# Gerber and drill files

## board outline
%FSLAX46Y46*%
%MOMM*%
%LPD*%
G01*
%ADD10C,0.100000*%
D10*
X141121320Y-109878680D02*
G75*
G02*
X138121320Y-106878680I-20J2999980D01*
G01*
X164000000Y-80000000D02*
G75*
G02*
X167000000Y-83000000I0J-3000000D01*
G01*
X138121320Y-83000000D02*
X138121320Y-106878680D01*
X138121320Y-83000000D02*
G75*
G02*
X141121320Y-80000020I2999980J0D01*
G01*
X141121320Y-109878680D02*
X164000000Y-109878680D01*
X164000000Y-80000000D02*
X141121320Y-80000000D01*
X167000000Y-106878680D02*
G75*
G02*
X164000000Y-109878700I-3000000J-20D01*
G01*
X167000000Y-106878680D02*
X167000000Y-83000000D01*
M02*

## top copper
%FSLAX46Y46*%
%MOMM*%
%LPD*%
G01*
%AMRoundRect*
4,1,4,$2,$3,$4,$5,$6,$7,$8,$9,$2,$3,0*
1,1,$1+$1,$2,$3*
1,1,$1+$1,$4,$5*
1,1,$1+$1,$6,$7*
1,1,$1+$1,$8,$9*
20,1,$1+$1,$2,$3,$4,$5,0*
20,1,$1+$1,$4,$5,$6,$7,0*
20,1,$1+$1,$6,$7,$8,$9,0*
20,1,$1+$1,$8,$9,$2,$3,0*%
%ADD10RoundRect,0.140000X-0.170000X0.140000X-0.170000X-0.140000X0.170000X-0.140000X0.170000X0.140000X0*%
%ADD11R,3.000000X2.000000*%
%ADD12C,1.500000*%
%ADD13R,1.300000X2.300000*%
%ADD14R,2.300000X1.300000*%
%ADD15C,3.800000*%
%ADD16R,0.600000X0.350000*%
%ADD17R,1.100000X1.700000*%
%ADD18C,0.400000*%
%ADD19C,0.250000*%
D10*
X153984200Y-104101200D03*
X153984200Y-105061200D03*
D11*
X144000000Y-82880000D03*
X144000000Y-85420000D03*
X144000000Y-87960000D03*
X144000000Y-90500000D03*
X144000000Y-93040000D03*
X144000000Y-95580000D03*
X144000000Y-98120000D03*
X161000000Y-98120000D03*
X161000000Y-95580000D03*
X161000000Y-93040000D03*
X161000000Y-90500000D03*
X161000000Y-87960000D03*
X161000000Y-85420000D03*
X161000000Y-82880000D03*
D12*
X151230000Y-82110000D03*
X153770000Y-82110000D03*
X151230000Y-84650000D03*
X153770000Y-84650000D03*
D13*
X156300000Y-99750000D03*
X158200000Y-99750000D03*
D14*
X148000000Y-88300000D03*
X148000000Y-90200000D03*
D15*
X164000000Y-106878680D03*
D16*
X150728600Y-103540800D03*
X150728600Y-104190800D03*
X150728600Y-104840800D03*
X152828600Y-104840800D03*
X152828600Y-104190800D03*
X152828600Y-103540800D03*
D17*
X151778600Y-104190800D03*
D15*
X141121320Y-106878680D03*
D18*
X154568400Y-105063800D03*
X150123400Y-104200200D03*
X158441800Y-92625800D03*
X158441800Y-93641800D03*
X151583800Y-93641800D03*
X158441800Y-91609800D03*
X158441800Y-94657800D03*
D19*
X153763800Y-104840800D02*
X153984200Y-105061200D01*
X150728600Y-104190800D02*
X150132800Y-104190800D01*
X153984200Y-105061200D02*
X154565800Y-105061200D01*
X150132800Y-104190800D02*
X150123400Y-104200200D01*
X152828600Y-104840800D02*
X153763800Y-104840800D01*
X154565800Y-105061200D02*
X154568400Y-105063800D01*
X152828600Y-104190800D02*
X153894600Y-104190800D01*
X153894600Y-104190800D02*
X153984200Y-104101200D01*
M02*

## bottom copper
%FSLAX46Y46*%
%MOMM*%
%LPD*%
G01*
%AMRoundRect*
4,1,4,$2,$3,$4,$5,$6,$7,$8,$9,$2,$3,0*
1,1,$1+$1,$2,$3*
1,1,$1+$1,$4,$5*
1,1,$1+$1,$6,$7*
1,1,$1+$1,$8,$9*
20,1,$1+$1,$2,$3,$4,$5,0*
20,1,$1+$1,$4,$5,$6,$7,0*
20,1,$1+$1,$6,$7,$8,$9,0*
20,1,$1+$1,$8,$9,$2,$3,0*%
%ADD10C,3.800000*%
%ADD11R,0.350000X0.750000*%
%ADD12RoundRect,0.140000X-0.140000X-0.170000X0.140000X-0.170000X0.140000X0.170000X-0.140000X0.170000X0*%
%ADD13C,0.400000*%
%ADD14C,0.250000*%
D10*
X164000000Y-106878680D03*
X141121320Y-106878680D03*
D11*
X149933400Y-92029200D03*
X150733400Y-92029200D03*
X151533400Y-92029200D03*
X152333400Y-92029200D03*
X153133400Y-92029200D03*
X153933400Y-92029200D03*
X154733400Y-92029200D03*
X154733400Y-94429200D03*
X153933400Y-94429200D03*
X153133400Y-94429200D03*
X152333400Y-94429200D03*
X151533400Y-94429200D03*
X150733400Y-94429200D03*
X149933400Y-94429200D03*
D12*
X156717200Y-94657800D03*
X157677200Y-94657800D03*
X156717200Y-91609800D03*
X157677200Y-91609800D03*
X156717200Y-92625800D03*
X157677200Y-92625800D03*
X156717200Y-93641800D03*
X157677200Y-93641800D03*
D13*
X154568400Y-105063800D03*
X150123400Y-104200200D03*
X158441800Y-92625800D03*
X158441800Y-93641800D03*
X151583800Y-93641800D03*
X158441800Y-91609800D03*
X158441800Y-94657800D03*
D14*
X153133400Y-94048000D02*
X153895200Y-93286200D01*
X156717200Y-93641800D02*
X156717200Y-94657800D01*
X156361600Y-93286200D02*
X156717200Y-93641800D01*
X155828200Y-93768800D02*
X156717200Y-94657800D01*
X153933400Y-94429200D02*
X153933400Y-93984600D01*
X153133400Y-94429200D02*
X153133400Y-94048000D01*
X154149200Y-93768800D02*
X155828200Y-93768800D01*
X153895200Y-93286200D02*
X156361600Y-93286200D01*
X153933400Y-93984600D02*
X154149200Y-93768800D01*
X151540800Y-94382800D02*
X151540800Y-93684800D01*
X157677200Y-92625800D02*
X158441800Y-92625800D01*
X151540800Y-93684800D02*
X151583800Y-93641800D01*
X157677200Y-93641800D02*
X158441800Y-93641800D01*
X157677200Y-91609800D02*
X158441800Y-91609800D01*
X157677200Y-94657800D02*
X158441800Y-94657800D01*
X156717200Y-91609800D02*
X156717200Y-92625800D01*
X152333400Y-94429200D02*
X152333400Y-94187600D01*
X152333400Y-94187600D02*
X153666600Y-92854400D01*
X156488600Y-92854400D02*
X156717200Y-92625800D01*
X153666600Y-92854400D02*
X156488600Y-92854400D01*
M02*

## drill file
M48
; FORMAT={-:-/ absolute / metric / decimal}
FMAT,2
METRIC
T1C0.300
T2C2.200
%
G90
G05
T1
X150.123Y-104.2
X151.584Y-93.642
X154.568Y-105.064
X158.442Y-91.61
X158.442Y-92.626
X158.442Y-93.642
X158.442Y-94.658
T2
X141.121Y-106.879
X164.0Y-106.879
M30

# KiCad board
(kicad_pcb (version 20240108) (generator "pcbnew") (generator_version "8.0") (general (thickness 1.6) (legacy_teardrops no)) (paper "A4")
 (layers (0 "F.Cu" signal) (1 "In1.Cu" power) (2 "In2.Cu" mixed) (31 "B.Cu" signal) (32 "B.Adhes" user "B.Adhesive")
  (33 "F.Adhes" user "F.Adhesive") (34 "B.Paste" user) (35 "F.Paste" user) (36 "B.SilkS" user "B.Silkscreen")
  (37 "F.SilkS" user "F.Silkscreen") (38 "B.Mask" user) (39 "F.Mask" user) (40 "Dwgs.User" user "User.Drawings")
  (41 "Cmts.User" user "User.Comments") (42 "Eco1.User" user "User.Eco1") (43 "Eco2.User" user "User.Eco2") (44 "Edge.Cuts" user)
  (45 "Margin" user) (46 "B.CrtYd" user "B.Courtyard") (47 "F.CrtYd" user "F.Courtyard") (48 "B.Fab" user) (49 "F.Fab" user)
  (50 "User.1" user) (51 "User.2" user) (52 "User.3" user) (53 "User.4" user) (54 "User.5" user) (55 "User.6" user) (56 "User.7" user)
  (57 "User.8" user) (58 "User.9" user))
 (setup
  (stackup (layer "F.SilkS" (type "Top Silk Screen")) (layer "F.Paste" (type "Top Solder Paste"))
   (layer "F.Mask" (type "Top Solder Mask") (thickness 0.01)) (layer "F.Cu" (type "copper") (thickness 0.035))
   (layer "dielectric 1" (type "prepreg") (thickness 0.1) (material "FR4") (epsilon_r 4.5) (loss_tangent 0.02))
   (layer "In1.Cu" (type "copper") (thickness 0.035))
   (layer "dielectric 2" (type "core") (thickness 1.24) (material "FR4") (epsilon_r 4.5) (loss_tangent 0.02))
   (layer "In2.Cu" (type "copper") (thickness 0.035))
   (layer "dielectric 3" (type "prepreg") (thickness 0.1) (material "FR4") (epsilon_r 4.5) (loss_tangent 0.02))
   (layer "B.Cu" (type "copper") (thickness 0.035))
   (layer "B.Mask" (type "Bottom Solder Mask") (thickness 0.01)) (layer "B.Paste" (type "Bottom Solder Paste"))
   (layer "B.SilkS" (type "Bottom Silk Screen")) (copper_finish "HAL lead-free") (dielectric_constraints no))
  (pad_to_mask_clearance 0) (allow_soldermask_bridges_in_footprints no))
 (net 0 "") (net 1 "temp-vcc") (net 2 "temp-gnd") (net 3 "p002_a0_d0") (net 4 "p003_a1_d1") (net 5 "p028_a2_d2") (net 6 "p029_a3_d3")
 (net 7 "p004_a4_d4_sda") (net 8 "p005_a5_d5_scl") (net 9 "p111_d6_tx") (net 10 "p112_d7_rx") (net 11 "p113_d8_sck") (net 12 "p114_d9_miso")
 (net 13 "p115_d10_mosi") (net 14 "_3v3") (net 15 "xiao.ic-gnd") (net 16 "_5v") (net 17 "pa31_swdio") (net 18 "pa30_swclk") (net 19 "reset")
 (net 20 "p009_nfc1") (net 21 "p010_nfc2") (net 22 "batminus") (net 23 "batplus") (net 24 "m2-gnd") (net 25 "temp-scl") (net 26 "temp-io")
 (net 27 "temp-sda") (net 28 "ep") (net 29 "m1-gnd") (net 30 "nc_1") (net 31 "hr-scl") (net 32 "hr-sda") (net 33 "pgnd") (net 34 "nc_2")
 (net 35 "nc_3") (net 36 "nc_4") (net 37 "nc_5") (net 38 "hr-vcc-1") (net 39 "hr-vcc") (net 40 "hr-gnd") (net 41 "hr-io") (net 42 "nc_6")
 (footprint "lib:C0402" (layer "F.Cu") (at 153.9842 104.5812 -90)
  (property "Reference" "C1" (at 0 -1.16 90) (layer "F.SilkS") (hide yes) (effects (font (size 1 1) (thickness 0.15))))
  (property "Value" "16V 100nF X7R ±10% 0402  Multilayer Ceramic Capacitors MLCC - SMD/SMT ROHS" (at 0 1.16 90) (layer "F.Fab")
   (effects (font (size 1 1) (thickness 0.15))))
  (pad "1" smd roundrect (at -0.48 0 270) (size 0.56 0.62) (layers "F.Cu" "F.Paste" "F.Mask") (roundrect_rratio 0.25) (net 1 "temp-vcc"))
  (pad "2" smd roundrect (at 0.48 0 270) (size 0.56 0.62) (layers "F.Cu" "F.Paste" "F.Mask") (roundrect_rratio 0.25) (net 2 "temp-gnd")))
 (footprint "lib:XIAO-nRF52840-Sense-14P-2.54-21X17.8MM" (layer "F.Cu") (at 152.5 90.5)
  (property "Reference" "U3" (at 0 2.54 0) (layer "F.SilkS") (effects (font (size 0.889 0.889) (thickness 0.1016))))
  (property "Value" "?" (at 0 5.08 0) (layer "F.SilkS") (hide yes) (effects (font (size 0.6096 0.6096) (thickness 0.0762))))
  (pad "1" smd rect (at -8.5 -7.62) (size 3 2) (layers "F.Cu" "F.Paste" "F.Mask") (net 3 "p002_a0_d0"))
  (pad "2" smd rect (at -8.5 -5.08) (size 3 2) (layers "F.Cu" "F.Paste" "F.Mask") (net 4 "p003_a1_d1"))
  (pad "3" smd rect (at -8.5 -2.54) (size 3 2) (layers "F.Cu" "F.Paste" "F.Mask") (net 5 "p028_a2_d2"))
  (pad "4" smd rect (at -8.5 0) (size 3 2) (layers "F.Cu" "F.Paste" "F.Mask") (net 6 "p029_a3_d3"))
  (pad "5" smd rect (at -8.5 2.54) (size 3 2) (layers "F.Cu" "F.Paste" "F.Mask") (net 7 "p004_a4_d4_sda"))
  (pad "6" smd rect (at -8.5 5.08 180) (size 3 2) (layers "F.Cu" "F.Paste" "F.Mask") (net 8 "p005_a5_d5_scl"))
  (pad "7" smd rect (at -8.5 7.62) (size 3 2) (layers "F.Cu" "F.Paste" "F.Mask") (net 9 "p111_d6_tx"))
  (pad "8" smd rect (at 8.5 7.62) (size 3 2) (layers "F.Cu" "F.Paste" "F.Mask") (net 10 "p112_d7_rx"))
  (pad "9" smd rect (at 8.5 5.08) (size 3 2) (layers "F.Cu" "F.Paste" "F.Mask") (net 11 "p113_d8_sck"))
  (pad "10" smd rect (at 8.5 2.54) (size 3 2) (layers "F.Cu" "F.Paste" "F.Mask") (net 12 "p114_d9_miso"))
  (pad "11" smd rect (at 8.5 0) (size 3 2) (layers "F.Cu" "F.Paste" "F.Mask") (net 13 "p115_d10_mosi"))
  (pad "12" smd rect (at 8.5 -2.54) (size 3 2) (layers "F.Cu" "F.Paste" "F.Mask") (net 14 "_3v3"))
  (pad "13" smd rect (at 8.5 -5.08) (size 3 2) (layers "F.Cu" "F.Paste" "F.Mask") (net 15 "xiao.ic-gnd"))
  (pad "14" smd rect (at 8.5 -7.62) (size 3 2) (layers "F.Cu" "F.Paste" "F.Mask") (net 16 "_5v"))
  (pad "15" smd circle (at -1.27 -8.39 90) (size 1.5 1.5) (layers "F.Cu" "F.Paste" "F.Mask") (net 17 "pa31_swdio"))
  (pad "16" smd circle (at 1.27 -8.39 90) (size 1.5 1.5) (layers "F.Cu" "F.Paste" "F.Mask") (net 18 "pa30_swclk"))
  (pad "17" smd circle (at -1.27 -5.85 90) (size 1.5 1.5) (layers "F.Cu" "F.Paste" "F.Mask") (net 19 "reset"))
  (pad "18" smd circle (at 1.27 -5.85 90) (size 1.5 1.5) (layers "F.Cu" "F.Paste" "F.Mask") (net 15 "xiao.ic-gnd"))
  (pad "19" smd rect (at 3.8 9.25 90) (size 2.3 1.3) (layers "F.Cu" "F.Paste" "F.Mask") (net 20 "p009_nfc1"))
  (pad "20" smd rect (at 5.7 9.25 90) (size 2.3 1.3) (layers "F.Cu" "F.Paste" "F.Mask") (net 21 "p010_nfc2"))
  (pad "21" smd rect (at -4.5 -2.2 180) (size 2.3 1.3) (layers "F.Cu" "F.Paste" "F.Mask") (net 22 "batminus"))
  (pad "22" smd rect (at -4.5 -0.3 180) (size 2.3 1.3) (layers "F.Cu" "F.Paste" "F.Mask") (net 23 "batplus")))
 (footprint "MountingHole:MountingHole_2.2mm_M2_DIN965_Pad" (layer "F.Cu") (at 164 106.87868)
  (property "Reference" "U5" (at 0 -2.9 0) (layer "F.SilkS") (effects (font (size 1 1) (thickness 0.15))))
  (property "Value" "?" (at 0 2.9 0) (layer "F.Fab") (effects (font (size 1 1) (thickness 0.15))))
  (pad "1" thru_hole circle (at 0 0) (size 3.8 3.8) (drill 2.2) (layers "*.Cu" "*.Mask") (remove_unused_layers no) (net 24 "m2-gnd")))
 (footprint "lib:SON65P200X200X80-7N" (layer "F.Cu") (at 151.7786 104.1908)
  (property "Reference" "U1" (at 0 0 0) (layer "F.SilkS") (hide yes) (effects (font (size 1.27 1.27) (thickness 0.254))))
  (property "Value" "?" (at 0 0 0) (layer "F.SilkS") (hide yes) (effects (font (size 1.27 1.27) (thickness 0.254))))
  (pad "1" smd rect (at -1.05 -0.65 90) (size 0.35 0.6) (layers "F.Cu" "F.Paste" "F.Mask") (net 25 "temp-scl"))
  (pad "2" smd rect (at -1.05 0 90) (size 0.35 0.6) (layers "F.Cu" "F.Paste" "F.Mask") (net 2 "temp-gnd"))
  (pad "3" smd rect (at -1.05 0.65 90) (size 0.35 0.6) (layers "F.Cu" "F.Paste" "F.Mask") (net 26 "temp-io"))
  (pad "4" smd rect (at 1.05 0.65 90) (size 0.35 0.6) (layers "F.Cu" "F.Paste" "F.Mask") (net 2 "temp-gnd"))
  (pad "5" smd rect (at 1.05 0 90) (size 0.35 0.6) (layers "F.Cu" "F.Paste" "F.Mask") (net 1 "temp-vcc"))
  (pad "6" smd rect (at 1.05 -0.65 90) (size 0.35 0.6) (layers "F.Cu" "F.Paste" "F.Mask") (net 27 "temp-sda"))
  (pad "7" smd rect (at 0 0) (size 1.1 1.7) (layers "F.Cu" "F.Paste" "F.Mask") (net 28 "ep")))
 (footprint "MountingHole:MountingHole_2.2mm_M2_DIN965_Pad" (layer "F.Cu") (at 141.12132 106.87868)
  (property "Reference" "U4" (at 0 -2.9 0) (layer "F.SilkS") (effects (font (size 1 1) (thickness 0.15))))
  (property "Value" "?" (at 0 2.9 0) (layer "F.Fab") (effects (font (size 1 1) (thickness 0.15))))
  (pad "1" thru_hole circle (at 0 0) (size 3.8 3.8) (drill 2.2) (layers "*.Cu" "*.Mask") (remove_unused_layers no) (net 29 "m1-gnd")))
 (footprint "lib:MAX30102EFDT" (layer "B.Cu") (at 152.3334 93.2292 -90)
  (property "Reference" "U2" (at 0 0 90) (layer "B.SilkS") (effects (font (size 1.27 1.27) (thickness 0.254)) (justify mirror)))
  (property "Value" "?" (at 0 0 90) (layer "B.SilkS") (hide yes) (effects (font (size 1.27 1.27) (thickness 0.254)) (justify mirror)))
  (pad "1" smd rect (at -1.2 2.4 180) (size 0.35 0.75) (layers "B.Cu" "B.Paste" "B.Mask") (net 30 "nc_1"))
  (pad "2" smd rect (at -1.2 1.6 180) (size 0.35 0.75) (layers "B.Cu" "B.Paste" "B.Mask") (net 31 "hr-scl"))
  (pad "3" smd rect (at -1.2 0.8 180) (size 0.35 0.75) (layers "B.Cu" "B.Paste" "B.Mask") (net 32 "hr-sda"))
  (pad "4" smd rect (at -1.2 0 180) (size 0.35 0.75) (layers "B.Cu" "B.Paste" "B.Mask") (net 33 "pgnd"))
  (pad "5" smd rect (at -1.2 -0.8 180) (size 0.35 0.75) (layers "B.Cu" "B.Paste" "B.Mask") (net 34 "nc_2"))
  (pad "6" smd rect (at -1.2 -1.6 180) (size 0.35 0.75) (layers "B.Cu" "B.Paste" "B.Mask") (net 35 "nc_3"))
  (pad "7" smd rect (at -1.2 -2.4 180) (size 0.35 0.75) (layers "B.Cu" "B.Paste" "B.Mask") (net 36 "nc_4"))
  (pad "8" smd rect (at 1.2 -2.4 180) (size 0.35 0.75) (layers "B.Cu" "B.Paste" "B.Mask") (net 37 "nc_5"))
  (pad "9" smd rect (at 1.2 -1.6 180) (size 0.35 0.75) (layers "B.Cu" "B.Paste" "B.Mask") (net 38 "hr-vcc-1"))
  (pad "10" smd rect (at 1.2 -0.8 180) (size 0.35 0.75) (layers "B.Cu" "B.Paste" "B.Mask") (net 38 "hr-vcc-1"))
  (pad "11" smd rect (at 1.2 0 180) (size 0.35 0.75) (layers "B.Cu" "B.Paste" "B.Mask") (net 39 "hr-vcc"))
  (pad "12" smd rect (at 1.2 0.8 180) (size 0.35 0.75) (layers "B.Cu" "B.Paste" "B.Mask") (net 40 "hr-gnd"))
  (pad "13" smd rect (at 1.2 1.6 180) (size 0.35 0.75) (layers "B.Cu" "B.Paste" "B.Mask") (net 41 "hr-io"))
  (pad "14" smd rect (at 1.2 2.4 180) (size 0.35 0.75) (layers "B.Cu" "B.Paste" "B.Mask") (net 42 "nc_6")))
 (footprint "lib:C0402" (layer "B.Cu") (at 157.1972 94.6578)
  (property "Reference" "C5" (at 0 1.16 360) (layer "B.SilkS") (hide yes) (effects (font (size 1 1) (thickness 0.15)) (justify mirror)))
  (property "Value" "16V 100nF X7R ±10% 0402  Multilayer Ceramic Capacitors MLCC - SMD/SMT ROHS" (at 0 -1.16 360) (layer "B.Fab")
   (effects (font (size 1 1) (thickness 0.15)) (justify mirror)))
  (pad "1" smd roundrect (at -0.48 0) (size 0.56 0.62) (layers "B.Cu" "B.Paste" "B.Mask") (roundrect_rratio 0.25) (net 38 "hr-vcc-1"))
  (pad "2" smd roundrect (at 0.48 0) (size 0.56 0.62) (layers "B.Cu" "B.Paste" "B.Mask") (roundrect_rratio 0.25) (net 40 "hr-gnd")))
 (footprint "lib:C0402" (layer "B.Cu") (at 157.1972 91.6098)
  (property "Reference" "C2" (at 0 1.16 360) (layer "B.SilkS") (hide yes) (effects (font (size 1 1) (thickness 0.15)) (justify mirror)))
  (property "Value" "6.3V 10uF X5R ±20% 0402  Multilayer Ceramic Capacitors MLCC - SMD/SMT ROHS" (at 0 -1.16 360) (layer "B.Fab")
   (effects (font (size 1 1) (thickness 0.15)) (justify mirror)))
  (pad "1" smd roundrect (at -0.48 0) (size 0.56 0.62) (layers "B.Cu" "B.Paste" "B.Mask") (roundrect_rratio 0.25) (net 39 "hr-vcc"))
  (pad "2" smd roundrect (at 0.48 0) (size 0.56 0.62) (layers "B.Cu" "B.Paste" "B.Mask") (roundrect_rratio 0.25) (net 40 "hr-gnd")))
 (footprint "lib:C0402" (layer "B.Cu") (at 157.1972 92.6258)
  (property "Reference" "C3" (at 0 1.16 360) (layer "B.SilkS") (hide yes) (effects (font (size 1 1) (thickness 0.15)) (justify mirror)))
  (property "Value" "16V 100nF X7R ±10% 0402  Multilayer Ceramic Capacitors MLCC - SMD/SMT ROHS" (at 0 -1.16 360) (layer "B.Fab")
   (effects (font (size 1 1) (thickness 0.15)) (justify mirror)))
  (pad "1" smd roundrect (at -0.48 0) (size 0.56 0.62) (layers "B.Cu" "B.Paste" "B.Mask") (roundrect_rratio 0.25) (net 39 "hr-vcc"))
  (pad "2" smd roundrect (at 0.48 0) (size 0.56 0.62) (layers "B.Cu" "B.Paste" "B.Mask") (roundrect_rratio 0.25) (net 40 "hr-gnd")))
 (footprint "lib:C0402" (layer "B.Cu") (at 157.1972 93.6418)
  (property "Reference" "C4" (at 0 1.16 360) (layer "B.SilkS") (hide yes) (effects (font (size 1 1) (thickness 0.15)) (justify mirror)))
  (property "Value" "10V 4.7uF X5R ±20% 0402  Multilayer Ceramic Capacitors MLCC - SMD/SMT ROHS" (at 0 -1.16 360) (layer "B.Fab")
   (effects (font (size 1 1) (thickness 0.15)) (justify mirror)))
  (pad "1" smd roundrect (at -0.48 0) (size 0.56 0.62) (layers "B.Cu" "B.Paste" "B.Mask") (roundrect_rratio 0.25) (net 38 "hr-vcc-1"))
  (pad "2" smd roundrect (at 0.48 0) (size 0.56 0.62) (layers "B.Cu" "B.Paste" "B.Mask") (roundrect_rratio 0.25) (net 40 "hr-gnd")))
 (gr_arc (start 141.12132 109.87868) (mid 139 109) (end 138.12132 106.87868) (stroke (width 0.1) (type default)) (layer "Edge.Cuts"))
 (gr_arc (start 164 80) (mid 166.12132 80.87868) (end 167 83) (stroke (width 0.1) (type default)) (layer "Edge.Cuts"))
 (gr_line (start 138.12132 83) (end 138.12132 106.87868) (stroke (width 0.1) (type default)) (layer "Edge.Cuts"))
 (gr_arc (start 138.12132 83) (mid 139 80.87868) (end 141.12132 80) (stroke (width 0.1) (type default)) (layer "Edge.Cuts"))
 (gr_line (start 141.12132 109.87868) (end 164 109.87868) (stroke (width 0.1) (type default)) (layer "Edge.Cuts"))
 (gr_line (start 164 80) (end 141.12132 80) (stroke (width 0.1) (type default)) (layer "Edge.Cuts"))
 (gr_arc (start 167 106.87868) (mid 166.12132 109) (end 164 109.87868) (stroke (width 0.1) (type default)) (layer "Edge.Cuts"))
 (gr_line (start 167 106.87868) (end 167 83) (stroke (width 0.1) (type default)) (layer "Edge.Cuts"))
 (segment (start 153.7638 104.8408) (end 153.9842 105.0612) (width 0.25) (layer "F.Cu") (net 2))
 (segment (start 150.7286 104.1908) (end 150.1328 104.1908) (width 0.25) (layer "F.Cu") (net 2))
 (segment (start 153.9842 105.0612) (end 154.5658 105.0612) (width 0.25) (layer "F.Cu") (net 2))
 (segment (start 150.1328 104.1908) (end 150.1234 104.2002) (width 0.25) (layer "F.Cu") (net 2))
 (segment (start 152.8286 104.8408) (end 153.7638 104.8408) (width 0.25) (layer "F.Cu") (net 2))
 (segment (start 154.5658 105.0612) (end 154.5684 105.0638) (width 0.25) (layer "F.Cu") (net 2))
 (via (at 154.5684 105.0638) (size 0.4) (drill 0.3) (layers "F.Cu" "B.Cu") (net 2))
 (via (at 150.1234 104.2002) (size 0.4) (drill 0.3) (layers "F.Cu" "B.Cu") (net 2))
 (segment (start 152.8286 104.1908) (end 153.8946 104.1908) (width 0.25) (layer "F.Cu") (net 1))
 (segment (start 153.8946 104.1908) (end 153.9842 104.1012) (width 0.25) (layer "F.Cu") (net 1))
 (segment (start 153.1334 94.048) (end 153.8952 93.2862) (width 0.25) (layer "B.Cu") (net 38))
 (segment (start 156.7172 93.6418) (end 156.7172 94.6578) (width 0.25) (layer "B.Cu") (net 38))
 (segment (start 156.3616 93.2862) (end 156.7172 93.6418) (width 0.25) (layer "B.Cu") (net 38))
 (segment (start 155.8282 93.7688) (end 156.7172 94.6578) (width 0.25) (layer "B.Cu") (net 38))
 (segment (start 153.9334 94.4292) (end 153.9334 93.9846) (width 0.25) (layer "B.Cu") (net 38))
 (segment (start 153.1334 94.4292) (end 153.1334 94.048) (width 0.25) (layer "B.Cu") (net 38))
 (segment (start 154.1492 93.7688) (end 155.8282 93.7688) (width 0.25) (layer "B.Cu") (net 38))
 (segment (start 153.8952 93.2862) (end 156.3616 93.2862) (width 0.25) (layer "B.Cu") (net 38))
 (segment (start 153.9334 93.9846) (end 154.1492 93.7688) (width 0.25) (layer "B.Cu") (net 38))
 (via (at 158.4418 92.6258) (size 0.4) (drill 0.3) (layers "F.Cu" "B.Cu") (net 40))
 (via (at 158.4418 93.6418) (size 0.4) (drill 0.3) (layers "F.Cu" "B.Cu") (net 40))
 (via (at 151.5838 93.6418) (size 0.4) (drill 0.3) (layers "F.Cu" "B.Cu") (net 40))
 (via (at 158.4418 91.6098) (size 0.4) (drill 0.3) (layers "F.Cu" "B.Cu") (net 40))
 (via (at 158.4418 94.6578) (size 0.4) (drill 0.3) (layers "F.Cu" "B.Cu") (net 40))
 (segment (start 151.5408 94.3828) (end 151.5408 93.6848) (width 0.25) (layer "B.Cu") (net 40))
 (segment (start 157.6772 92.6258) (end 158.4418 92.6258) (width 0.25) (layer "B.Cu") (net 40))
 (segment (start 151.5408 93.6848) (end 151.5838 93.6418) (width 0.25) (layer "B.Cu") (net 40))
 (segment (start 157.6772 93.6418) (end 158.4418 93.6418) (width 0.25) (layer "B.Cu") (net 40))
 (segment (start 157.6772 91.6098) (end 158.4418 91.6098) (width 0.25) (layer "B.Cu") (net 40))
 (segment (start 157.6772 94.6578) (end 158.4418 94.6578) (width 0.25) (layer "B.Cu") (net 40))
 (segment (start 156.7172 91.6098) (end 156.7172 92.6258) (width 0.25) (layer "B.Cu") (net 39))
 (segment (start 152.3334 94.4292) (end 152.3334 94.1876) (width 0.25) (layer "B.Cu") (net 39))
 (segment (start 152.3334 94.1876) (end 153.6666 92.8544) (width 0.25) (layer "B.Cu") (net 39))
 (segment (start 156.4886 92.8544) (end 156.7172 92.6258) (width 0.25) (layer "B.Cu") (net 39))
 (segment (start 153.6666 92.8544) (end 156.4886 92.8544) (width 0.25) (layer "B.Cu") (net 39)))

